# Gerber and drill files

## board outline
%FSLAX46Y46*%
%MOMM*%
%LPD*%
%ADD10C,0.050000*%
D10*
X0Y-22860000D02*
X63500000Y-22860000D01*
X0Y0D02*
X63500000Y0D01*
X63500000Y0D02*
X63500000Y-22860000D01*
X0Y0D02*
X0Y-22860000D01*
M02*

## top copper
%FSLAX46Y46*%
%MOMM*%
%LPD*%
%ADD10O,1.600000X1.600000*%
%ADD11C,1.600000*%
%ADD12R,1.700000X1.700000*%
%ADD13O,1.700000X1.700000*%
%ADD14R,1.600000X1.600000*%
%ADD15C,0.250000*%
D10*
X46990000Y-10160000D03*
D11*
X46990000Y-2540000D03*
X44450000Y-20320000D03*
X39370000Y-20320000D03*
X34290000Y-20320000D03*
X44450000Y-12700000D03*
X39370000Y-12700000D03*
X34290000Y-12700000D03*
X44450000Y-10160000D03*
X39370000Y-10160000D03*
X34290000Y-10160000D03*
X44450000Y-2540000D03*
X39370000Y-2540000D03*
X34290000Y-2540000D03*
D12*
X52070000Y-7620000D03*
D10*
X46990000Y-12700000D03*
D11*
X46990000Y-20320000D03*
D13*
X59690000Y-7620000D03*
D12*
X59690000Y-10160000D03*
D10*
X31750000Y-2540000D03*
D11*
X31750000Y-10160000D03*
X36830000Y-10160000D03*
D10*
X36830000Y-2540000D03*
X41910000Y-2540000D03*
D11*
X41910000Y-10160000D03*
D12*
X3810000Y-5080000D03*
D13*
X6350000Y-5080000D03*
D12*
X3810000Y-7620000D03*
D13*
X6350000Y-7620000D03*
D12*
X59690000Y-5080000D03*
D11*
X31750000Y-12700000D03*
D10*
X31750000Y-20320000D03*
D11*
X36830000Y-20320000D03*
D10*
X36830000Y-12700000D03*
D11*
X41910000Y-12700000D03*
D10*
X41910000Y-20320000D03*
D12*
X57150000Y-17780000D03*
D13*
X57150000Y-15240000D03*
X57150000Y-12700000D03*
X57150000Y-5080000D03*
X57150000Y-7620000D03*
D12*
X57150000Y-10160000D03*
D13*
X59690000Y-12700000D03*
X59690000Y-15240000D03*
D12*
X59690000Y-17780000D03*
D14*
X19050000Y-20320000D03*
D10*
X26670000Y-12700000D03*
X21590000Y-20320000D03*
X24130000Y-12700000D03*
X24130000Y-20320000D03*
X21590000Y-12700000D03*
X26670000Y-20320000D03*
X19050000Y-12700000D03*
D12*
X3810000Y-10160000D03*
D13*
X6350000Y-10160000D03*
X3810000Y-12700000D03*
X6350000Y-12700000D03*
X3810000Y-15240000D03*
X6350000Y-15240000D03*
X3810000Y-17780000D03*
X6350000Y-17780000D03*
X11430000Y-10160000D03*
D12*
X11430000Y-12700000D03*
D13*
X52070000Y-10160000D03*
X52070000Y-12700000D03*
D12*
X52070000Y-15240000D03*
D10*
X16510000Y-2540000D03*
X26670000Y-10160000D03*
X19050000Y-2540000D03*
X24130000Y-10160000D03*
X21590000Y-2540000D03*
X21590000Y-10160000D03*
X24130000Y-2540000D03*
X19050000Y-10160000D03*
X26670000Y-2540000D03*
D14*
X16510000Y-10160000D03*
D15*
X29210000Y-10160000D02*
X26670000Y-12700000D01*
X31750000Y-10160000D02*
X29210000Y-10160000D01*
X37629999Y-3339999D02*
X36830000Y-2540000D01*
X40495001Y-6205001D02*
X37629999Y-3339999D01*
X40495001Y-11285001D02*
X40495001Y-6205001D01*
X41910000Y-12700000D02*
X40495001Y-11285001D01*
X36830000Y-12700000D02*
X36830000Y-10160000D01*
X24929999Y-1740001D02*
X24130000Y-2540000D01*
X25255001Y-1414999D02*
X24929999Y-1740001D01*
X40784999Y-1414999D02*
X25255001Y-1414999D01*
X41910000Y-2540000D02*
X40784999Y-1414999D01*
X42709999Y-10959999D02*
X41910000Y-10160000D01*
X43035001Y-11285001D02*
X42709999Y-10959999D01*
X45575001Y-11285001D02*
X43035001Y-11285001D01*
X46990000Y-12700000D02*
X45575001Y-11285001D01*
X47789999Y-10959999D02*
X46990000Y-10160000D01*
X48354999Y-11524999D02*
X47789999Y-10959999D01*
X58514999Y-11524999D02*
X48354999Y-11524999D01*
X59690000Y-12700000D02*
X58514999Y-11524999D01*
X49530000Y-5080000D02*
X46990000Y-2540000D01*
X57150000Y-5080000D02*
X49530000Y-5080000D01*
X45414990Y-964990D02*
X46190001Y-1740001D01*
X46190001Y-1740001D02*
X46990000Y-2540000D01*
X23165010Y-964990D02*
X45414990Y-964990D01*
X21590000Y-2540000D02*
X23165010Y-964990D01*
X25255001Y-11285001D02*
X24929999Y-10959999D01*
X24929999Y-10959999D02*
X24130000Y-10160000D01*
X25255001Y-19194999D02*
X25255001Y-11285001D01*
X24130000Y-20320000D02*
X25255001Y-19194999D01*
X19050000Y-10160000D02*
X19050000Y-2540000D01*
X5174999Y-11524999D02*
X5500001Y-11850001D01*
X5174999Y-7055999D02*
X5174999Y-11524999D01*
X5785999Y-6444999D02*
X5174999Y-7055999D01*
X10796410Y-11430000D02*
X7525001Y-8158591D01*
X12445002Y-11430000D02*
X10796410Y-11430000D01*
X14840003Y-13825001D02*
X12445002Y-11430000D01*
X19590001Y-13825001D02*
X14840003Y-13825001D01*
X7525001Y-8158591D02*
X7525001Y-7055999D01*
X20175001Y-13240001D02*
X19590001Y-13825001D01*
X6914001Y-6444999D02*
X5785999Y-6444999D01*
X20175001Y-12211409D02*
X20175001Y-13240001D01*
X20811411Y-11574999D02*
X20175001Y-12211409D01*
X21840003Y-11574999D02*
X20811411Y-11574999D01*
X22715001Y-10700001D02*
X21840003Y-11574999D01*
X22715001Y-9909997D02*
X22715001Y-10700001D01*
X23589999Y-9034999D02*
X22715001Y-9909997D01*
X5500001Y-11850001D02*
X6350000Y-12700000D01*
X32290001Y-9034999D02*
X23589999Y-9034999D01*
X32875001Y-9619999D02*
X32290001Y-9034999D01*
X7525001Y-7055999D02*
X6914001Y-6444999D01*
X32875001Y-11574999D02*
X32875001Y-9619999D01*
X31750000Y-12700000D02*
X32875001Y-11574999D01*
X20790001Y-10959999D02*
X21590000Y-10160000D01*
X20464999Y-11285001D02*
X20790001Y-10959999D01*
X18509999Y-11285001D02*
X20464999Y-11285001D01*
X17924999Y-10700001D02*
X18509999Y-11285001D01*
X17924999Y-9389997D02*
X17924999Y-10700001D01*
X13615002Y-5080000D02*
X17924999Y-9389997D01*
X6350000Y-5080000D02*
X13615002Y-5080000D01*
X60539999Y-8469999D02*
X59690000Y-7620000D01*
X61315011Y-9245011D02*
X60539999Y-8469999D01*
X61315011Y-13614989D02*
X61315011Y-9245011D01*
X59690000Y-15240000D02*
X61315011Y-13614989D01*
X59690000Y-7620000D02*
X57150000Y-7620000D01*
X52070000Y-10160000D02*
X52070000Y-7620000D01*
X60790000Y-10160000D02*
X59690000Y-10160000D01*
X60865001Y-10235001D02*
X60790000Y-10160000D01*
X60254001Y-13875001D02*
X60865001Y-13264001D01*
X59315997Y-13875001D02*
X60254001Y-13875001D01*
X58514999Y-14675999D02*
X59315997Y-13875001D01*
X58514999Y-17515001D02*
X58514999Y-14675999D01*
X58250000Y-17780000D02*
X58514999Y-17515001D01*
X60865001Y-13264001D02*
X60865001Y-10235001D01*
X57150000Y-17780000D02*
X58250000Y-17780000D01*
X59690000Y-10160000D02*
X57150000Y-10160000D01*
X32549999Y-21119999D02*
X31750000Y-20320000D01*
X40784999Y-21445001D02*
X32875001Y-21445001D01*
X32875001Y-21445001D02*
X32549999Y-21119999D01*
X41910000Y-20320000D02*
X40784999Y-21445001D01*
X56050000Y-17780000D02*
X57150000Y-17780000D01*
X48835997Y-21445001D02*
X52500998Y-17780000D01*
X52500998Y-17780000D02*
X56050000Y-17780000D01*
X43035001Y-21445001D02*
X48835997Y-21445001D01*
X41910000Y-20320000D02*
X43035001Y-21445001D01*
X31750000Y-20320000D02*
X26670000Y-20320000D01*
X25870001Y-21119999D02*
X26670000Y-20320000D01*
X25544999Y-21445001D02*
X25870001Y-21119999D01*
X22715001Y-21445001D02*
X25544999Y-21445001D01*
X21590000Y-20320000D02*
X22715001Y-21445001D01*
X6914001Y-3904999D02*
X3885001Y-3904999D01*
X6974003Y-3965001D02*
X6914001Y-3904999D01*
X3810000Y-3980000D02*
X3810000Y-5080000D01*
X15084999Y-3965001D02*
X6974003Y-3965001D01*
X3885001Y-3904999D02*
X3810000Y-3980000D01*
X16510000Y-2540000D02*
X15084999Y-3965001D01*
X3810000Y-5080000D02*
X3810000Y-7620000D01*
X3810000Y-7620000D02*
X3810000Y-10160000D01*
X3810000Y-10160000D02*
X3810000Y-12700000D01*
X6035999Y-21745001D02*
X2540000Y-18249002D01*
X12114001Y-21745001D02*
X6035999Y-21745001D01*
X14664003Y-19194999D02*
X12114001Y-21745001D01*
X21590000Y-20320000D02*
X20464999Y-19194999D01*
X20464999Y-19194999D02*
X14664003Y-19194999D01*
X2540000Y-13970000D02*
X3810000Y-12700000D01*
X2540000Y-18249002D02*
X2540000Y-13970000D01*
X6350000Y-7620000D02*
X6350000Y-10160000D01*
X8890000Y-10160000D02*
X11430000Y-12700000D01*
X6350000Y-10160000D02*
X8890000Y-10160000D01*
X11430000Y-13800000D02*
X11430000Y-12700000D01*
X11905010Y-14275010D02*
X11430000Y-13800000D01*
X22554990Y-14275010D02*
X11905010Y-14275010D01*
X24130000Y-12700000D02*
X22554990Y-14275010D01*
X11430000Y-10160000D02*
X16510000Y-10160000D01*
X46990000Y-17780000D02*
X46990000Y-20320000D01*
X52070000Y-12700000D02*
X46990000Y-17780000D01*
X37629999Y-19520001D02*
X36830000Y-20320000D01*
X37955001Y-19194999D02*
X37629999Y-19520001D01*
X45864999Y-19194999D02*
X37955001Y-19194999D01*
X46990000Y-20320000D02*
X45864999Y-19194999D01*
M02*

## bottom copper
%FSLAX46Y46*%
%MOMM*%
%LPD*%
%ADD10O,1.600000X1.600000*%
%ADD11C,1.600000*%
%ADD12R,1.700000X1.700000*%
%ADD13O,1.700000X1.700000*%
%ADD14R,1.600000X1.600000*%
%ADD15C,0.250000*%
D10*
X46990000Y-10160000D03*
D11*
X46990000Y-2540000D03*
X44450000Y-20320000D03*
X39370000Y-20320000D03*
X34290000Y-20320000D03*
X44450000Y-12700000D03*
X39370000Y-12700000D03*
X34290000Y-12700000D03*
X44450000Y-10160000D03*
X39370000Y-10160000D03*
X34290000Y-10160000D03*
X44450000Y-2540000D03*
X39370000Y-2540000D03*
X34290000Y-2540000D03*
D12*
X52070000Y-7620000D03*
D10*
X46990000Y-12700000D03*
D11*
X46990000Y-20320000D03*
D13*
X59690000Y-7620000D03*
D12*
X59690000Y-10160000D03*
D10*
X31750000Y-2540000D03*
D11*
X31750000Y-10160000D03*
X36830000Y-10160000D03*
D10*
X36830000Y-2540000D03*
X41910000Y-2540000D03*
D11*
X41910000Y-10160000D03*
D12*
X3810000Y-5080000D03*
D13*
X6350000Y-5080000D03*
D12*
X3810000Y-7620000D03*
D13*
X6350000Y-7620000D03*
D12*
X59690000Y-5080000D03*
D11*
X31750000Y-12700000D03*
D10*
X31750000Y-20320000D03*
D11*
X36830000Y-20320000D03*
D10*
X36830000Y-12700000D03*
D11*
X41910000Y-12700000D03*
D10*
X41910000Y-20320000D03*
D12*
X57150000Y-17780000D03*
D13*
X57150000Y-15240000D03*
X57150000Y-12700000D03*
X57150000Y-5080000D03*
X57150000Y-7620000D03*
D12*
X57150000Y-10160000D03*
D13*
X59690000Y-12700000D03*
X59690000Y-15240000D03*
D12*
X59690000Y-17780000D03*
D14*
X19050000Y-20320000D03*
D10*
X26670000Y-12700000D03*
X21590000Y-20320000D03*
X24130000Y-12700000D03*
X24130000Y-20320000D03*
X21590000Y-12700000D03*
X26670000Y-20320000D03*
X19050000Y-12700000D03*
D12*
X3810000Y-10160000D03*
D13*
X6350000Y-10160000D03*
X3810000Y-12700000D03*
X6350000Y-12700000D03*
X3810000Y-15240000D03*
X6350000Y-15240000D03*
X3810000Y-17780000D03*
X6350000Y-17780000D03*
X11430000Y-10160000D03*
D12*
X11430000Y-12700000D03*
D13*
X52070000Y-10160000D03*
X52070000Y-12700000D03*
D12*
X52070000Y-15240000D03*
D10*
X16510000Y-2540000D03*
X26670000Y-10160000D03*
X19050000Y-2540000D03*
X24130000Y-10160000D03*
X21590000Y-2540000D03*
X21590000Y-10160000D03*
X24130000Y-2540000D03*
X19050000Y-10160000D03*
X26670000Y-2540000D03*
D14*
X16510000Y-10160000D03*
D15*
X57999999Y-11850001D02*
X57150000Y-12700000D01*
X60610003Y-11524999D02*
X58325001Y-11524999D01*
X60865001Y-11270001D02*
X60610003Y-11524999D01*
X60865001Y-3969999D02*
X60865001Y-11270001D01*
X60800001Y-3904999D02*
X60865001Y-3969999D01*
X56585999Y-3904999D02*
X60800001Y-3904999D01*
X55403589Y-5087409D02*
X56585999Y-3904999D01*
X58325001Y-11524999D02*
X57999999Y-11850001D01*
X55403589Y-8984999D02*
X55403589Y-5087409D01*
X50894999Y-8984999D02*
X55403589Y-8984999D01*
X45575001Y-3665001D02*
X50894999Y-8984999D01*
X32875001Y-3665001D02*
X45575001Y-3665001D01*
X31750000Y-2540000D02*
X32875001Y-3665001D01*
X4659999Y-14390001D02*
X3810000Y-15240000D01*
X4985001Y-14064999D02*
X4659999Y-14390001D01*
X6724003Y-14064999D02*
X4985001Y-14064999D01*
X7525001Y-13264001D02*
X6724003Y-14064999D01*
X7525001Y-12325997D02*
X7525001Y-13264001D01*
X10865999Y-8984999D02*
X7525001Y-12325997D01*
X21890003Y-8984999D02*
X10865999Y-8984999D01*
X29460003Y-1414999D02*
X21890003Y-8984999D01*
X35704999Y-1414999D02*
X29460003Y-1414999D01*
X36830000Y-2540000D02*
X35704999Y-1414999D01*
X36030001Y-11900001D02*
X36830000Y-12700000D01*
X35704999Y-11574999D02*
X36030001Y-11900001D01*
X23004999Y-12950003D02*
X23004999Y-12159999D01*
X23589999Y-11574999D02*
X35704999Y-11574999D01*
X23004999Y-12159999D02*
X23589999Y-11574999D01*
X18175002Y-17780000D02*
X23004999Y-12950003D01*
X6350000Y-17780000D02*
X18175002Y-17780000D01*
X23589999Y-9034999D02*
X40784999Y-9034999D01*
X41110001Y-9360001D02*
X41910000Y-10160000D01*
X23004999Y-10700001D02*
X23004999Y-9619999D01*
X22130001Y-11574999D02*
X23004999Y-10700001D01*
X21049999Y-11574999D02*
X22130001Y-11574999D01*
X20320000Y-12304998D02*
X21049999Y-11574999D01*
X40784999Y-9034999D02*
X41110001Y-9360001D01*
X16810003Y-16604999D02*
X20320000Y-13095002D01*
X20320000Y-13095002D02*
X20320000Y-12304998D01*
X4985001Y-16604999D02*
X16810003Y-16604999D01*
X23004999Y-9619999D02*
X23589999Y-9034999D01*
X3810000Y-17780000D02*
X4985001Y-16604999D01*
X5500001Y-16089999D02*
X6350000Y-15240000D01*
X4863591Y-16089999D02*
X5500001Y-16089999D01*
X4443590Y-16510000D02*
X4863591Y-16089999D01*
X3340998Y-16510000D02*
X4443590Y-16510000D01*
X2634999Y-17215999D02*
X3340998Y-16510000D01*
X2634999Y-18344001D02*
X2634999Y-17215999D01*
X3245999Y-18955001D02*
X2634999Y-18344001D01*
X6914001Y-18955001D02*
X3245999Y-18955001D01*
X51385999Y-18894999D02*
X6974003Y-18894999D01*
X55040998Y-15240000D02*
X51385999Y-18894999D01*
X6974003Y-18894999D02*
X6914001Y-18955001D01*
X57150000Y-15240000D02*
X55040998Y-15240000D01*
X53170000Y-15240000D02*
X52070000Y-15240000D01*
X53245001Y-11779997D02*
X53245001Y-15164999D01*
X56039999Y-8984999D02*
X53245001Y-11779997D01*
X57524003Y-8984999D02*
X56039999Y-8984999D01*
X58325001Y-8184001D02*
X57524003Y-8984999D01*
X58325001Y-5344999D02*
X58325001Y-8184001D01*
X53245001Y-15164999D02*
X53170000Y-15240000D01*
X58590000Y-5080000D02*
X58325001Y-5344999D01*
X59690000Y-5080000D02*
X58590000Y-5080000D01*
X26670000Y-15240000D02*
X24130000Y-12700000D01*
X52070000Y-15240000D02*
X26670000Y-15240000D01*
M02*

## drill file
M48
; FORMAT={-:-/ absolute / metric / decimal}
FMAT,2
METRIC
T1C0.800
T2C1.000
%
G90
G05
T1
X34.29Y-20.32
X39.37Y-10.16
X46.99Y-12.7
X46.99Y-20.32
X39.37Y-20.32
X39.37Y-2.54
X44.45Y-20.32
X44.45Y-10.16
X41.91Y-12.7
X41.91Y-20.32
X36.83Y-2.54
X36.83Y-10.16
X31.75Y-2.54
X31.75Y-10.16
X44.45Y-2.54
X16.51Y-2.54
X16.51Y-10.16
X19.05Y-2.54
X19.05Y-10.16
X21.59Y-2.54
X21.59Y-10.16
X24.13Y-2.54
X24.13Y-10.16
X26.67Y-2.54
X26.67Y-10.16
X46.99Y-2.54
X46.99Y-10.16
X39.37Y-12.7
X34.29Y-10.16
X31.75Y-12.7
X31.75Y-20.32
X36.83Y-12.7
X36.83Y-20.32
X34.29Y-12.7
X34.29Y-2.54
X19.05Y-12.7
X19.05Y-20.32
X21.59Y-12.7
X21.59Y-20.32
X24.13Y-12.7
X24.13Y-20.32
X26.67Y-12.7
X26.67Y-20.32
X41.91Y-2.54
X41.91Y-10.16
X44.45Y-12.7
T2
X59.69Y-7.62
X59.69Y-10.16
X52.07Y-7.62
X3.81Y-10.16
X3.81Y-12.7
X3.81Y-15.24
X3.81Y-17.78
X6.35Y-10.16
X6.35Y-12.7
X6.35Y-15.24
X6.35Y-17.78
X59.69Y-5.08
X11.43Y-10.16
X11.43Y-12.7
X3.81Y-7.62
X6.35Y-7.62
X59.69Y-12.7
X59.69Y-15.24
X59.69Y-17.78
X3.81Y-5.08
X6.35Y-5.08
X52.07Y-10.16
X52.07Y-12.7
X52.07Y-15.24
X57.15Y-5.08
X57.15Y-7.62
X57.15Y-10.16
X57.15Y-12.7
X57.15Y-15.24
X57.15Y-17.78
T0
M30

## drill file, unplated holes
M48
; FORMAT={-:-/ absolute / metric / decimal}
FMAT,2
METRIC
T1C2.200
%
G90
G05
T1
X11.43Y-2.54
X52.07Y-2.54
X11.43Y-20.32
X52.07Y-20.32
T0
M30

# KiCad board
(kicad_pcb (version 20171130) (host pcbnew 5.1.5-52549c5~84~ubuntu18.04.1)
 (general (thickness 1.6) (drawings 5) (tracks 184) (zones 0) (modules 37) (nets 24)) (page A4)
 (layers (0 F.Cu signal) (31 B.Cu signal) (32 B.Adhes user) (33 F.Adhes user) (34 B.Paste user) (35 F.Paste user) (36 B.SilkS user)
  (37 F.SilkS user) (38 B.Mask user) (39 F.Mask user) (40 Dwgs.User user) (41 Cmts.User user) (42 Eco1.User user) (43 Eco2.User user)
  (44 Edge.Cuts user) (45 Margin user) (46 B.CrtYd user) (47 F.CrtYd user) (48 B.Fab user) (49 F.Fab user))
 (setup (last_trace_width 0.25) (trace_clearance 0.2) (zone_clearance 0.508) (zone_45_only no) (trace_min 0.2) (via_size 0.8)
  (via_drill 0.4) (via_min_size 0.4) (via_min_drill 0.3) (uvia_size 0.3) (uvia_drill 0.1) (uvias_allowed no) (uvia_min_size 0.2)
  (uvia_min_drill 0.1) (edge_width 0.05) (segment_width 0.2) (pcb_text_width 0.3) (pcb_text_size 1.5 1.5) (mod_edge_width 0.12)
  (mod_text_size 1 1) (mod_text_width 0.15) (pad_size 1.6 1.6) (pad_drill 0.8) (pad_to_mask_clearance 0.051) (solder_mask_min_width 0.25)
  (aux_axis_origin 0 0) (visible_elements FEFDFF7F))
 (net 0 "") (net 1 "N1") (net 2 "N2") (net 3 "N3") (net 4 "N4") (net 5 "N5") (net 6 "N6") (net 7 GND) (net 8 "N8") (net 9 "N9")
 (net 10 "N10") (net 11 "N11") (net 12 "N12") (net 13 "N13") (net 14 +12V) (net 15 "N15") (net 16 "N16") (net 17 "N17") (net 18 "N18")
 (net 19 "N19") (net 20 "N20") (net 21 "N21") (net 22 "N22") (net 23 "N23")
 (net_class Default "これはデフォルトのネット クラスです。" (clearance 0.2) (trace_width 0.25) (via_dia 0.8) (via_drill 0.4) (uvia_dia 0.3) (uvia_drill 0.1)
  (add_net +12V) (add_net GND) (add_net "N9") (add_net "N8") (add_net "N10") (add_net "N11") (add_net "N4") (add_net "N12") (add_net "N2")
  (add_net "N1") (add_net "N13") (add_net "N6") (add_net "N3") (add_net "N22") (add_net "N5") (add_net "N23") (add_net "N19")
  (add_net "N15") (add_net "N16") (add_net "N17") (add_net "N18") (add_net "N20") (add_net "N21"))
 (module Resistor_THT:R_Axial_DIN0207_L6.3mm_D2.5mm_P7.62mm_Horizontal (layer F.Cu) (at 46.99 2.54 270)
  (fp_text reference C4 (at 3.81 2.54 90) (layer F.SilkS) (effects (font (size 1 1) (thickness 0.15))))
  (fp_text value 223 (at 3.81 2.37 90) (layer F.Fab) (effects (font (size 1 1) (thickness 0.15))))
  (pad 2 thru_hole oval (at 7.62 0 270) (size 1.6 1.6) (drill 0.8) (layers *.Cu *.Mask) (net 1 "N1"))
  (pad 1 thru_hole circle (at 0 0 270) (size 1.6 1.6) (drill 0.8) (layers *.Cu *.Mask) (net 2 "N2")))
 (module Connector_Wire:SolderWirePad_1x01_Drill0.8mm (layer F.Cu) (at 44.45 20.32)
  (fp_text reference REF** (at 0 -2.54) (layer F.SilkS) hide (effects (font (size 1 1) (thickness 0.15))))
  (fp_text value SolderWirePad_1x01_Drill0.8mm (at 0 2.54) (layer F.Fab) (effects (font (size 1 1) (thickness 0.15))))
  (pad 1 thru_hole circle (at 0 0) (size 1.6 1.6) (drill 0.8) (layers *.Cu *.Mask)))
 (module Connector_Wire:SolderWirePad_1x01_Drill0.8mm (layer F.Cu) (at 39.37 20.32)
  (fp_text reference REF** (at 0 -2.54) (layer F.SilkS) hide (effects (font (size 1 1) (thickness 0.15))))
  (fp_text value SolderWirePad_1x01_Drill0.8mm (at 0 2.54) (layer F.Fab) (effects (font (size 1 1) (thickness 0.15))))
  (pad 1 thru_hole circle (at 0 0) (size 1.6 1.6) (drill 0.8) (layers *.Cu *.Mask)))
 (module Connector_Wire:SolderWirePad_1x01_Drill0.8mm (layer F.Cu) (at 34.29 20.32)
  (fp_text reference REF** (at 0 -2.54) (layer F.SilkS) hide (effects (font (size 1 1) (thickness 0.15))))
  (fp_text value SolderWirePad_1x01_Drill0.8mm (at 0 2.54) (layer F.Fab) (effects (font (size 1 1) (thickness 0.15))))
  (pad 1 thru_hole circle (at 0 0) (size 1.6 1.6) (drill 0.8) (layers *.Cu *.Mask)))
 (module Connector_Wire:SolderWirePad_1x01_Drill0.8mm (layer F.Cu) (at 44.45 12.7)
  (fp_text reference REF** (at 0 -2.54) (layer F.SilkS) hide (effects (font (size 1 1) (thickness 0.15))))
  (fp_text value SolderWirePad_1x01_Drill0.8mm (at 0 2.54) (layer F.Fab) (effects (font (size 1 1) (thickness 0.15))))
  (pad 1 thru_hole circle (at 0 0) (size 1.6 1.6) (drill 0.8) (layers *.Cu *.Mask)))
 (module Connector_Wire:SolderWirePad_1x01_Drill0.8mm (layer F.Cu) (at 39.37 12.7)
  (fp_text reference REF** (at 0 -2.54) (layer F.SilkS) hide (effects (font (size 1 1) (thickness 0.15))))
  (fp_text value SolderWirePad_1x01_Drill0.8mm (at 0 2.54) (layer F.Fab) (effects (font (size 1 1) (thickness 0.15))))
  (pad 1 thru_hole circle (at 0 0) (size 1.6 1.6) (drill 0.8) (layers *.Cu *.Mask)))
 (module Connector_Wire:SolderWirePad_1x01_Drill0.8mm (layer F.Cu) (at 34.29 12.7)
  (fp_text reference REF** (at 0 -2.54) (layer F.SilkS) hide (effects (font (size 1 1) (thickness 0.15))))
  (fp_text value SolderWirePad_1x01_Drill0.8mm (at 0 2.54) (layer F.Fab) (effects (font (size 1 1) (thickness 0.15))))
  (pad 1 thru_hole circle (at 0 0) (size 1.6 1.6) (drill 0.8) (layers *.Cu *.Mask)))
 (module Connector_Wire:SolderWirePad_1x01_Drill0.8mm (layer F.Cu) (at 44.45 10.16)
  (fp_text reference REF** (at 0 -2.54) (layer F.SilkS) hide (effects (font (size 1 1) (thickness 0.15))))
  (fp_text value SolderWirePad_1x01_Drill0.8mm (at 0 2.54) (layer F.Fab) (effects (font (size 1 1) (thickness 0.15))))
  (pad 1 thru_hole circle (at 0 0) (size 1.6 1.6) (drill 0.8) (layers *.Cu *.Mask)))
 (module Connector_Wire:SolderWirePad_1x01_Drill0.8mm (layer F.Cu) (at 39.37 10.16)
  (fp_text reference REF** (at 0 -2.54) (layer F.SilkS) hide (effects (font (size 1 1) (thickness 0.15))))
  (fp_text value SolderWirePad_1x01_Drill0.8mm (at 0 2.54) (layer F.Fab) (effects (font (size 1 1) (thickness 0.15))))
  (pad 1 thru_hole circle (at 0 0) (size 1.6 1.6) (drill 0.8) (layers *.Cu *.Mask)))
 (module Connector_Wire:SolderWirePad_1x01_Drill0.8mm (layer F.Cu) (at 34.29 10.16)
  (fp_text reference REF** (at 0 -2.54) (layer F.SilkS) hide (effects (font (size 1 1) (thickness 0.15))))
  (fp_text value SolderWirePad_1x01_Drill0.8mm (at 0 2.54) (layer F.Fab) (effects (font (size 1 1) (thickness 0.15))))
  (pad 1 thru_hole circle (at 0 0) (size 1.6 1.6) (drill 0.8) (layers *.Cu *.Mask)))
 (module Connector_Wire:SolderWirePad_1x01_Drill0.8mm (layer F.Cu) (at 44.45 2.54)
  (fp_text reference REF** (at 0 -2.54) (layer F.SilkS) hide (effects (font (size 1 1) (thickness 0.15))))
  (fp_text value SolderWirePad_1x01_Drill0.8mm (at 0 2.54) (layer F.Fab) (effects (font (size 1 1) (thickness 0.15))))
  (pad 1 thru_hole circle (at 0 0) (size 1.6 1.6) (drill 0.8) (layers *.Cu *.Mask)))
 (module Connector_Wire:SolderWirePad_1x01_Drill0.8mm (layer F.Cu) (at 39.37 2.54)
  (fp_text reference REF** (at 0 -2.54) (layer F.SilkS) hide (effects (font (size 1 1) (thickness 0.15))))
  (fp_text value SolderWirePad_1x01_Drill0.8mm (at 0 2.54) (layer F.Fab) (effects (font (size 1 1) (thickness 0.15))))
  (pad 1 thru_hole circle (at 0 0) (size 1.6 1.6) (drill 0.8) (layers *.Cu *.Mask)))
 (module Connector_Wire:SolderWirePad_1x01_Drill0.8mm (layer F.Cu) (at 34.29 2.54)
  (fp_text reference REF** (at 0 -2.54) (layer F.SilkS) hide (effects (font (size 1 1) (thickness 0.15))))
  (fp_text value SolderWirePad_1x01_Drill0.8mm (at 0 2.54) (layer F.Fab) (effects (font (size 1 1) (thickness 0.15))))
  (pad 1 thru_hole circle (at 0 0) (size 1.6 1.6) (drill 0.8) (layers *.Cu *.Mask)))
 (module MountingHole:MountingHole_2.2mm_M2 (layer F.Cu) (at 52.07 20.32)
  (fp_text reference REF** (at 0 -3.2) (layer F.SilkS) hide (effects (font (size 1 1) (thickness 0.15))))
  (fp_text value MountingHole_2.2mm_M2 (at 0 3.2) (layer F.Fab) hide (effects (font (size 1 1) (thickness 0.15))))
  (pad 1 np_thru_hole circle (at 0 0) (size 2.2 2.2) (drill 2.2) (layers *.Cu *.Mask)))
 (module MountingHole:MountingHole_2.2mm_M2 (layer F.Cu) (at 11.43 20.32)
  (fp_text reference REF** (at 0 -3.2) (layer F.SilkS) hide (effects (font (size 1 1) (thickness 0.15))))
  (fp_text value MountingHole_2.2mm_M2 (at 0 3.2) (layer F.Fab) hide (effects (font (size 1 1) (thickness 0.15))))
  (pad 1 np_thru_hole circle (at 0 0) (size 2.2 2.2) (drill 2.2) (layers *.Cu *.Mask)))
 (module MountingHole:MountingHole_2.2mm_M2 (layer F.Cu) (at 52.07 2.54)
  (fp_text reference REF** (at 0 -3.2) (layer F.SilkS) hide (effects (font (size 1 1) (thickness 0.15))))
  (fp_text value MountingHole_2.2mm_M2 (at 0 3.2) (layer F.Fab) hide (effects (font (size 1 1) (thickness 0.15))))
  (pad 1 np_thru_hole circle (at 0 0) (size 2.2 2.2) (drill 2.2) (layers *.Cu *.Mask)))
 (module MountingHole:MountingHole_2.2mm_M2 (layer F.Cu) (at 11.43 2.54)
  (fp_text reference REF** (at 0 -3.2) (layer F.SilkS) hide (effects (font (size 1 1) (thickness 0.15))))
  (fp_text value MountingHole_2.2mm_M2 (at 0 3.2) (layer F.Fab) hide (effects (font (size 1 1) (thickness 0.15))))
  (pad 1 np_thru_hole circle (at 0 0) (size 2.2 2.2) (drill 2.2) (layers *.Cu *.Mask)))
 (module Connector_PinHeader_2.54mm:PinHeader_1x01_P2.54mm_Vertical (layer F.Cu) (at 52.07 7.62)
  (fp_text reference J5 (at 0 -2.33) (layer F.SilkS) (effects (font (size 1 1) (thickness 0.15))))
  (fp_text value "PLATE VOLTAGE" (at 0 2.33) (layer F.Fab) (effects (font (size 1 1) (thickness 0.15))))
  (pad 1 thru_hole rect (at 0 0) (size 1.7 1.7) (drill 1) (layers *.Cu *.Mask) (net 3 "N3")))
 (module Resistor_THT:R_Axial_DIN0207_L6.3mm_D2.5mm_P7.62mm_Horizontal (layer F.Cu) (at 46.99 20.32 90)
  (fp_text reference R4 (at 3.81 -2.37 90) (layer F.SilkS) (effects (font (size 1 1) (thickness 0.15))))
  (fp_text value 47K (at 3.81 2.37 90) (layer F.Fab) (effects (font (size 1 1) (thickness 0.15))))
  (pad 2 thru_hole oval (at 7.62 0 90) (size 1.6 1.6) (drill 0.8) (layers *.Cu *.Mask) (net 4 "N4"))
  (pad 1 thru_hole circle (at 0 0 90) (size 1.6 1.6) (drill 0.8) (layers *.Cu *.Mask) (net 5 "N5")))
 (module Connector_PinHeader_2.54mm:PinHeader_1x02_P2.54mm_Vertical (layer F.Cu) (at 59.69 10.16 180)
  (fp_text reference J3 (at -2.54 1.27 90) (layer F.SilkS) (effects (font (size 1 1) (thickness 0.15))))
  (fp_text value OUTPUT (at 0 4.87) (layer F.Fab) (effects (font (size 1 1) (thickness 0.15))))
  (pad 2 thru_hole oval (at 0 2.54 180) (size 1.7 1.7) (drill 1) (layers *.Cu *.Mask) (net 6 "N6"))
  (pad 1 thru_hole rect (at 0 0 180) (size 1.7 1.7) (drill 1) (layers *.Cu *.Mask) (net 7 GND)))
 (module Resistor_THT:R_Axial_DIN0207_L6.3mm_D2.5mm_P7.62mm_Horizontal (layer F.Cu) (at 31.75 10.16 90)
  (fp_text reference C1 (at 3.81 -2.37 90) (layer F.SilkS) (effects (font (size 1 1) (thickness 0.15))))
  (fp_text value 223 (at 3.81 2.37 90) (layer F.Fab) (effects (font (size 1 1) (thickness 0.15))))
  (pad 2 thru_hole oval (at 7.62 0 90) (size 1.6 1.6) (drill 0.8) (layers *.Cu *.Mask) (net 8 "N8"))
  (pad 1 thru_hole circle (at 0 0 90) (size 1.6 1.6) (drill 0.8) (layers *.Cu *.Mask) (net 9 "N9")))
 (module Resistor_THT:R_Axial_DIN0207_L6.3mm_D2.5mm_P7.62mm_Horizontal (layer F.Cu) (at 36.83 10.16 90)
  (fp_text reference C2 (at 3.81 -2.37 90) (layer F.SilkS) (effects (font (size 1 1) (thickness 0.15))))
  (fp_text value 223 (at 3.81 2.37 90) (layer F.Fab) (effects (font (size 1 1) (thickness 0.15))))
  (pad 1 thru_hole circle (at 0 0 90) (size 1.6 1.6) (drill 0.8) (layers *.Cu *.Mask) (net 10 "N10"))
  (pad 2 thru_hole oval (at 7.62 0 90) (size 1.6 1.6) (drill 0.8) (layers *.Cu *.Mask) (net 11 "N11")))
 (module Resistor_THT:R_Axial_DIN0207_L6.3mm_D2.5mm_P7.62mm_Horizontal (layer F.Cu) (at 41.91 10.16 90)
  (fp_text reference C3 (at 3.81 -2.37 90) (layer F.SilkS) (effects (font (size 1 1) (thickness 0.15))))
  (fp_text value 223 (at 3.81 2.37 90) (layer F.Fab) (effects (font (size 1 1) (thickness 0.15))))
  (pad 2 thru_hole oval (at 7.62 0 90) (size 1.6 1.6) (drill 0.8) (layers *.Cu *.Mask) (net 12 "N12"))
  (pad 1 thru_hole circle (at 0 0 90) (size 1.6 1.6) (drill 0.8) (layers *.Cu *.Mask) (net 4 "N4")))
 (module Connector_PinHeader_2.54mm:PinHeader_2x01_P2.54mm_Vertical (layer F.Cu) (at 3.81 5.08)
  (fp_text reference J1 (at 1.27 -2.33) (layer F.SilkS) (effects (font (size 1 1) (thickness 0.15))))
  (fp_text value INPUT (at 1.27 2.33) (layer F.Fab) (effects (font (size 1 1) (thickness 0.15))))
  (pad 1 thru_hole rect (at 0 0) (size 1.7 1.7) (drill 1) (layers *.Cu *.Mask) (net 7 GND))
  (pad 2 thru_hole oval (at 2.54 0) (size 1.7 1.7) (drill 1) (layers *.Cu *.Mask) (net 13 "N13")))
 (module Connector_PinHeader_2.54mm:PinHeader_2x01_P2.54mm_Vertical (layer F.Cu) (at 3.81 7.62)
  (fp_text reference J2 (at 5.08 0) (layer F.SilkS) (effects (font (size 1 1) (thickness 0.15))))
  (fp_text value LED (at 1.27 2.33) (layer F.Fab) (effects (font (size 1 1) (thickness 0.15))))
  (pad 1 thru_hole rect (at 0 0) (size 1.7 1.7) (drill 1) (layers *.Cu *.Mask) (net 7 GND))
  (pad 2 thru_hole oval (at 2.54 0) (size 1.7 1.7) (drill 1) (layers *.Cu *.Mask) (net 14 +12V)))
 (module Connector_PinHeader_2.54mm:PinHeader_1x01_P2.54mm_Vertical (layer F.Cu) (at 59.69 5.08 180)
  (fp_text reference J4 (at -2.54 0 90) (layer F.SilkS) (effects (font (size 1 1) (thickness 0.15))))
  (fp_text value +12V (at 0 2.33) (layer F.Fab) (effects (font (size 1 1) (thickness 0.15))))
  (pad 1 thru_hole rect (at 0 0 180) (size 1.7 1.7) (drill 1) (layers *.Cu *.Mask) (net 14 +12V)))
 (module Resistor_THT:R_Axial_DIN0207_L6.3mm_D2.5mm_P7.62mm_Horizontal (layer F.Cu) (at 31.75 12.7 270)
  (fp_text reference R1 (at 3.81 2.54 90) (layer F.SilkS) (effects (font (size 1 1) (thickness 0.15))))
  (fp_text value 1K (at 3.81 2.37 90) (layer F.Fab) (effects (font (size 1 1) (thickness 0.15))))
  (pad 1 thru_hole circle (at 0 0 270) (size 1.6 1.6) (drill 0.8) (layers *.Cu *.Mask) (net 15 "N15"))
  (pad 2 thru_hole oval (at 7.62 0 270) (size 1.6 1.6) (drill 0.8) (layers *.Cu *.Mask) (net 7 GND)))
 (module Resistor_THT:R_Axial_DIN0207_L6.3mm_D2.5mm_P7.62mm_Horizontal (layer F.Cu) (at 36.83 20.32 90)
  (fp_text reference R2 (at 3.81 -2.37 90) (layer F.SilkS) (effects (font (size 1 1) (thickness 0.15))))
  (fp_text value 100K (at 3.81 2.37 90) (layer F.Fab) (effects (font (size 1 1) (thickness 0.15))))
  (pad 1 thru_hole circle (at 0 0 90) (size 1.6 1.6) (drill 0.8) (layers *.Cu *.Mask) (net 5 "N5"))
  (pad 2 thru_hole oval (at 7.62 0 90) (size 1.6 1.6) (drill 0.8) (layers *.Cu *.Mask) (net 10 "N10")))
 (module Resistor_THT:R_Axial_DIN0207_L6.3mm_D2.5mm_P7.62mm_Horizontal (layer F.Cu) (at 41.91 12.7 270)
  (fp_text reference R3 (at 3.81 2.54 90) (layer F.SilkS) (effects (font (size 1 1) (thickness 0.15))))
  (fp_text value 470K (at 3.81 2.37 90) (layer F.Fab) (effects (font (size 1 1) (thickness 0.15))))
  (pad 1 thru_hole circle (at 0 0 270) (size 1.6 1.6) (drill 0.8) (layers *.Cu *.Mask) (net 11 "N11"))
  (pad 2 thru_hole oval (at 7.62 0 270) (size 1.6 1.6) (drill 0.8) (layers *.Cu *.Mask) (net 7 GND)))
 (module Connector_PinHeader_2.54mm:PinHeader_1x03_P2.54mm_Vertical (layer F.Cu) (at 57.15 17.78 180)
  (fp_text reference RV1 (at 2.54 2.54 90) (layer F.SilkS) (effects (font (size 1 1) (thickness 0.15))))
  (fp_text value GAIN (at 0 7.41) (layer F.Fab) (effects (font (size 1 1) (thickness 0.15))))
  (pad 1 thru_hole rect (at 0 0 180) (size 1.7 1.7) (drill 1) (layers *.Cu *.Mask) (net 7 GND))
  (pad 2 thru_hole oval (at 0 2.54 180) (size 1.7 1.7) (drill 1) (layers *.Cu *.Mask) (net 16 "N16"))
  (pad 3 thru_hole oval (at 0 5.08 180) (size 1.7 1.7) (drill 1) (layers *.Cu *.Mask) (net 8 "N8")))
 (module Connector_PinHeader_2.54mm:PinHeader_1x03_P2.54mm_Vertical (layer F.Cu) (at 57.15 10.16 180)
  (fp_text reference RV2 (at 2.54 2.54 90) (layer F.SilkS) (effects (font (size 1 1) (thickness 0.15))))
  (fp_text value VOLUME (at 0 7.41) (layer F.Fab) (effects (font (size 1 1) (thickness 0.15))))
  (pad 3 thru_hole oval (at 0 5.08 180) (size 1.7 1.7) (drill 1) (layers *.Cu *.Mask) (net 2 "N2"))
  (pad 2 thru_hole oval (at 0 2.54 180) (size 1.7 1.7) (drill 1) (layers *.Cu *.Mask) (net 6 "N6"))
  (pad 1 thru_hole rect (at 0 0 180) (size 1.7 1.7) (drill 1) (layers *.Cu *.Mask) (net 7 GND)))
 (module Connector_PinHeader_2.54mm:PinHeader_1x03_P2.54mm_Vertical (layer F.Cu) (at 59.69 17.78 180)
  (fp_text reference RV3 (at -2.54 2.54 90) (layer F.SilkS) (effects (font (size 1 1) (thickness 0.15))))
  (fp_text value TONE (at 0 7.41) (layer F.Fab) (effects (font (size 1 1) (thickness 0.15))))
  (pad 3 thru_hole oval (at 0 5.08 180) (size 1.7 1.7) (drill 1) (layers *.Cu *.Mask) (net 1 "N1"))
  (pad 2 thru_hole oval (at 0 2.54 180) (size 1.7 1.7) (drill 1) (layers *.Cu *.Mask) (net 6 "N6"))
  (pad 1 thru_hole rect (at 0 0 180) (size 1.7 1.7) (drill 1) (layers *.Cu *.Mask) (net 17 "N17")))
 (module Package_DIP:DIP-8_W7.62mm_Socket (layer F.Cu) (at 19.05 20.32 90)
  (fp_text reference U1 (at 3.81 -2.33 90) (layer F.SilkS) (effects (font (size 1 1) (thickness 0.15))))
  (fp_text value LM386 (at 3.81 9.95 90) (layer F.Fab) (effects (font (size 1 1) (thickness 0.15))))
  (pad 1 thru_hole rect (at 0 0 90) (size 1.6 1.6) (drill 0.8) (layers *.Cu *.Mask) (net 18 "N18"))
  (pad 5 thru_hole oval (at 7.62 7.62 90) (size 1.6 1.6) (drill 0.8) (layers *.Cu *.Mask) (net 9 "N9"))
  (pad 2 thru_hole oval (at 0 2.54 90) (size 1.6 1.6) (drill 0.8) (layers *.Cu *.Mask) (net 7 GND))
  (pad 6 thru_hole oval (at 7.62 5.08 90) (size 1.6 1.6) (drill 0.8) (layers *.Cu *.Mask) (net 14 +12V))
  (pad 3 thru_hole oval (at 0 5.08 90) (size 1.6 1.6) (drill 0.8) (layers *.Cu *.Mask) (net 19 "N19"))
  (pad 7 thru_hole oval (at 7.62 2.54 90) (size 1.6 1.6) (drill 0.8) (layers *.Cu *.Mask) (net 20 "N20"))
  (pad 4 thru_hole oval (at 0 7.62 90) (size 1.6 1.6) (drill 0.8) (layers *.Cu *.Mask) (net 7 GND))
  (pad 8 thru_hole oval (at 7.62 0 90) (size 1.6 1.6) (drill 0.8) (layers *.Cu *.Mask) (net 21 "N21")))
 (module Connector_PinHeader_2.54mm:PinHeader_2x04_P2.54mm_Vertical (layer F.Cu) (at 3.81 10.16)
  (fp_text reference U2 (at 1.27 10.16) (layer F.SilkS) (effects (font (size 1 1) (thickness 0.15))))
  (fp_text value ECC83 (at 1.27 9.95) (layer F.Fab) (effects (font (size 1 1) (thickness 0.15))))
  (pad 4 thru_hole rect (at 0 0) (size 1.7 1.7) (drill 1) (layers *.Cu *.Mask) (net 7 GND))
  (pad 5 thru_hole oval (at 2.54 0) (size 1.7 1.7) (drill 1) (layers *.Cu *.Mask) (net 14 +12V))
  (pad 3 thru_hole oval (at 0 2.54) (size 1.7 1.7) (drill 1) (layers *.Cu *.Mask) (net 7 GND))
  (pad 8 thru_hole oval (at 2.54 2.54) (size 1.7 1.7) (drill 1) (layers *.Cu *.Mask) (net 15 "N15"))
  (pad 2 thru_hole oval (at 0 5.08) (size 1.7 1.7) (drill 1) (layers *.Cu *.Mask) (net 11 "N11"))
  (pad 7 thru_hole oval (at 2.54 5.08) (size 1.7 1.7) (drill 1) (layers *.Cu *.Mask) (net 16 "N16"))
  (pad 1 thru_hole oval (at 0 7.62) (size 1.7 1.7) (drill 1) (layers *.Cu *.Mask) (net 4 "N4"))
  (pad 6 thru_hole oval (at 2.54 7.62) (size 1.7 1.7) (drill 1) (layers *.Cu *.Mask) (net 10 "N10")))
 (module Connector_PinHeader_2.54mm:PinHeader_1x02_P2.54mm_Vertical (layer F.Cu) (at 11.43 12.7 180)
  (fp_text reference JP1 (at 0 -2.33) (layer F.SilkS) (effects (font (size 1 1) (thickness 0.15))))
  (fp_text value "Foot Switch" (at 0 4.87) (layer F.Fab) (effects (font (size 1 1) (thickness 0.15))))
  (pad 2 thru_hole oval (at 0 2.54 180) (size 1.7 1.7) (drill 1) (layers *.Cu *.Mask) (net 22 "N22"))
  (pad 1 thru_hole rect (at 0 0 180) (size 1.7 1.7) (drill 1) (layers *.Cu *.Mask) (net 14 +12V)))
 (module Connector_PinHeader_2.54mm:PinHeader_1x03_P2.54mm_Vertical (layer F.Cu) (at 52.07 15.24 180)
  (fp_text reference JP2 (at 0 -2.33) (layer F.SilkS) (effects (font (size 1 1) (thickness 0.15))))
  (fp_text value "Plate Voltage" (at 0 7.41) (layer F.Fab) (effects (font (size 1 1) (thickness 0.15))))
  (pad 3 thru_hole oval (at 0 5.08 180) (size 1.7 1.7) (drill 1) (layers *.Cu *.Mask) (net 3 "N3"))
  (pad 2 thru_hole oval (at 0 2.54 180) (size 1.7 1.7) (drill 1) (layers *.Cu *.Mask) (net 5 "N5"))
  (pad 1 thru_hole rect (at 0 0 180) (size 1.7 1.7) (drill 1) (layers *.Cu *.Mask) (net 14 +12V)))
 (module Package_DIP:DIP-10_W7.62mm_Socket (layer F.Cu) (at 16.51 10.16 90)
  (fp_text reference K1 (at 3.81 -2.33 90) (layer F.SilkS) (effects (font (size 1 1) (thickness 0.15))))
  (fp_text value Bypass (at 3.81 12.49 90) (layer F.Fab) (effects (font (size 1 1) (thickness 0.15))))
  (pad 10 thru_hole oval (at 7.62 0 90) (size 1.6 1.6) (drill 0.8) (layers *.Cu *.Mask) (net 7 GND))
  (pad 5 thru_hole oval (at 0 10.16 90) (size 1.6 1.6) (drill 0.8) (layers *.Cu *.Mask))
  (pad 9 thru_hole oval (at 7.62 2.54 90) (size 1.6 1.6) (drill 0.8) (layers *.Cu *.Mask) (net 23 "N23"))
  (pad 4 thru_hole oval (at 0 7.62 90) (size 1.6 1.6) (drill 0.8) (layers *.Cu *.Mask) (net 19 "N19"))
  (pad 8 thru_hole oval (at 7.62 5.08 90) (size 1.6 1.6) (drill 0.8) (layers *.Cu *.Mask) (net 2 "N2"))
  (pad 3 thru_hole oval (at 0 5.08 90) (size 1.6 1.6) (drill 0.8) (layers *.Cu *.Mask) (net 13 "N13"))
  (pad 7 thru_hole oval (at 7.62 7.62 90) (size 1.6 1.6) (drill 0.8) (layers *.Cu *.Mask) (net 12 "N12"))
  (pad 2 thru_hole oval (at 0 2.54 90) (size 1.6 1.6) (drill 0.8) (layers *.Cu *.Mask) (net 23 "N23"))
  (pad 6 thru_hole oval (at 7.62 10.16 90) (size 1.6 1.6) (drill 0.8) (layers *.Cu *.Mask))
  (pad 1 thru_hole rect (at 0 0 90) (size 1.6 1.6) (drill 0.8) (layers *.Cu *.Mask) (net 22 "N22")))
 (gr_line (start 0 22.86) (end 63.5 22.86) (layer Edge.Cuts) (width 0.05))
 (gr_line (start 0 0) (end 63.5 0) (layer Edge.Cuts) (width 0.05))
 (gr_line (start 63.5 0) (end 63.5 22.86) (layer Edge.Cuts) (width 0.05))
 (gr_line (start 0 0) (end 0 22.86) (layer Edge.Cuts) (width 0.05))
 (segment (start 57.999999 11.850001) (end 57.15 12.7) (width 0.25) (layer B.Cu) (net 8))
 (segment (start 60.610003 11.524999) (end 58.325001 11.524999) (width 0.25) (layer B.Cu) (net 8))
 (segment (start 60.865001 11.270001) (end 60.610003 11.524999) (width 0.25) (layer B.Cu) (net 8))
 (segment (start 60.865001 3.969999) (end 60.865001 11.270001) (width 0.25) (layer B.Cu) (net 8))
 (segment (start 60.800001 3.904999) (end 60.865001 3.969999) (width 0.25) (layer B.Cu) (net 8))
 (segment (start 56.585999 3.904999) (end 60.800001 3.904999) (width 0.25) (layer B.Cu) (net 8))
 (segment (start 55.403589 5.087409) (end 56.585999 3.904999) (width 0.25) (layer B.Cu) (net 8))
 (segment (start 58.325001 11.524999) (end 57.999999 11.850001) (width 0.25) (layer B.Cu) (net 8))
 (segment (start 55.403589 8.984999) (end 55.403589 5.087409) (width 0.25) (layer B.Cu) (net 8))
 (segment (start 50.894999 8.984999) (end 55.403589 8.984999) (width 0.25) (layer B.Cu) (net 8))
 (segment (start 45.575001 3.665001) (end 50.894999 8.984999) (width 0.25) (layer B.Cu) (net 8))
 (segment (start 32.875001 3.665001) (end 45.575001 3.665001) (width 0.25) (layer B.Cu) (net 8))
 (segment (start 31.75 2.54) (end 32.875001 3.665001) (width 0.25) (layer B.Cu) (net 8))
 (segment (start 29.21 10.16) (end 26.67 12.7) (width 0.25) (layer F.Cu) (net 9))
 (segment (start 31.75 10.16) (end 29.21 10.16) (width 0.25) (layer F.Cu) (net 9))
 (segment (start 37.629999 3.339999) (end 36.83 2.54) (width 0.25) (layer F.Cu) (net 11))
 (segment (start 40.495001 6.205001) (end 37.629999 3.339999) (width 0.25) (layer F.Cu) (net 11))
 (segment (start 40.495001 11.285001) (end 40.495001 6.205001) (width 0.25) (layer F.Cu) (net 11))
 (segment (start 41.91 12.7) (end 40.495001 11.285001) (width 0.25) (layer F.Cu) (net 11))
 (segment (start 4.659999 14.390001) (end 3.81 15.24) (width 0.25) (layer B.Cu) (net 11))
 (segment (start 4.985001 14.064999) (end 4.659999 14.390001) (width 0.25) (layer B.Cu) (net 11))
 (segment (start 6.724003 14.064999) (end 4.985001 14.064999) (width 0.25) (layer B.Cu) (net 11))
 (segment (start 7.525001 13.264001) (end 6.724003 14.064999) (width 0.25) (layer B.Cu) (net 11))
 (segment (start 7.525001 12.325997) (end 7.525001 13.264001) (width 0.25) (layer B.Cu) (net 11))
 (segment (start 10.865999 8.984999) (end 7.525001 12.325997) (width 0.25) (layer B.Cu) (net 11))
 (segment (start 21.890003 8.984999) (end 10.865999 8.984999) (width 0.25) (layer B.Cu) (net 11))
 (segment (start 29.460003 1.414999) (end 21.890003 8.984999) (width 0.25) (layer B.Cu) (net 11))
 (segment (start 35.704999 1.414999) (end 29.460003 1.414999) (width 0.25) (layer B.Cu) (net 11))
 (segment (start 36.83 2.54) (end 35.704999 1.414999) (width 0.25) (layer B.Cu) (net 11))
 (segment (start 36.83 12.7) (end 36.83 10.16) (width 0.25) (layer F.Cu) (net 10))
 (segment (start 36.030001 11.900001) (end 36.83 12.7) (width 0.25) (layer B.Cu) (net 10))
 (segment (start 35.704999 11.574999) (end 36.030001 11.900001) (width 0.25) (layer B.Cu) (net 10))
 (segment (start 23.004999 12.950003) (end 23.004999 12.159999) (width 0.25) (layer B.Cu) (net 10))
 (segment (start 23.589999 11.574999) (end 35.704999 11.574999) (width 0.25) (layer B.Cu) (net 10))
 (segment (start 23.004999 12.159999) (end 23.589999 11.574999) (width 0.25) (layer B.Cu) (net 10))
 (segment (start 18.175002 17.78) (end 23.004999 12.950003) (width 0.25) (layer B.Cu) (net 10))
 (segment (start 6.35 17.78) (end 18.175002 17.78) (width 0.25) (layer B.Cu) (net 10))
 (segment (start 24.929999 1.740001) (end 24.13 2.54) (width 0.25) (layer F.Cu) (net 12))
 (segment (start 25.255001 1.414999) (end 24.929999 1.740001) (width 0.25) (layer F.Cu) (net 12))
 (segment (start 40.784999 1.414999) (end 25.255001 1.414999) (width 0.25) (layer F.Cu) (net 12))
 (segment (start 41.91 2.54) (end 40.784999 1.414999) (width 0.25) (layer F.Cu) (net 12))
 (segment (start 42.709999 10.959999) (end 41.91 10.16) (width 0.25) (layer F.Cu) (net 4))
 (segment (start 43.035001 11.285001) (end 42.709999 10.959999) (width 0.25) (layer F.Cu) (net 4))
 (segment (start 45.575001 11.285001) (end 43.035001 11.285001) (width 0.25) (layer F.Cu) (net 4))
 (segment (start 46.99 12.7) (end 45.575001 11.285001) (width 0.25) (layer F.Cu) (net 4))
 (segment (start 23.589999 9.034999) (end 40.784999 9.034999) (width 0.25) (layer B.Cu) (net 4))
 (segment (start 41.110001 9.360001) (end 41.91 10.16) (width 0.25) (layer B.Cu) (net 4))
 (segment (start 23.004999 10.700001) (end 23.004999 9.619999) (width 0.25) (layer B.Cu) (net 4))
 (segment (start 22.130001 11.574999) (end 23.004999 10.700001) (width 0.25) (layer B.Cu) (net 4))
 (segment (start 21.049999 11.574999) (end 22.130001 11.574999) (width 0.25) (layer B.Cu) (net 4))
 (segment (start 20.32 12.304998) (end 21.049999 11.574999) (width 0.25) (layer B.Cu) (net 4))
 (segment (start 40.784999 9.034999) (end 41.110001 9.360001) (width 0.25) (layer B.Cu) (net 4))
 (segment (start 16.810003 16.604999) (end 20.32 13.095002) (width 0.25) (layer B.Cu) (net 4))
 (segment (start 20.32 13.095002) (end 20.32 12.304998) (width 0.25) (layer B.Cu) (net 4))
 (segment (start 4.985001 16.604999) (end 16.810003 16.604999) (width 0.25) (layer B.Cu) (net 4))
 (segment (start 23.004999 9.619999) (end 23.589999 9.034999) (width 0.25) (layer B.Cu) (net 4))
 (segment (start 3.81 17.78) (end 4.985001 16.604999) (width 0.25) (layer B.Cu) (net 4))
 (segment (start 47.789999 10.959999) (end 46.99 10.16) (width 0.25) (layer F.Cu) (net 1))
 (segment (start 48.354999 11.524999) (end 47.789999 10.959999) (width 0.25) (layer F.Cu) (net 1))
 (segment (start 58.514999 11.524999) (end 48.354999 11.524999) (width 0.25) (layer F.Cu) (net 1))
 (segment (start 59.69 12.7) (end 58.514999 11.524999) (width 0.25) (layer F.Cu) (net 1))
 (segment (start 49.53 5.08) (end 46.99 2.54) (width 0.25) (layer F.Cu) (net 2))
 (segment (start 57.15 5.08) (end 49.53 5.08) (width 0.25) (layer F.Cu) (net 2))
 (segment (start 45.41499 0.96499) (end 46.190001 1.740001) (width 0.25) (layer F.Cu) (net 2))
 (segment (start 46.190001 1.740001) (end 46.99 2.54) (width 0.25) (layer F.Cu) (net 2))
 (segment (start 23.16501 0.96499) (end 45.41499 0.96499) (width 0.25) (layer F.Cu) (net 2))
 (segment (start 21.59 2.54) (end 23.16501 0.96499) (width 0.25) (layer F.Cu) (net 2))
 (segment (start 25.255001 11.285001) (end 24.929999 10.959999) (width 0.25) (layer F.Cu) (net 19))
 (segment (start 24.929999 10.959999) (end 24.13 10.16) (width 0.25) (layer F.Cu) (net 19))
 (segment (start 25.255001 19.194999) (end 25.255001 11.285001) (width 0.25) (layer F.Cu) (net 19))
 (segment (start 24.13 20.32) (end 25.255001 19.194999) (width 0.25) (layer F.Cu) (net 19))
 (segment (start 19.05 10.16) (end 19.05 2.54) (width 0.25) (layer F.Cu) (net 23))
 (segment (start 5.174999 11.524999) (end 5.500001 11.850001) (width 0.25) (layer F.Cu) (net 15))
 (segment (start 5.174999 7.055999) (end 5.174999 11.524999) (width 0.25) (layer F.Cu) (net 15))
 (segment (start 5.785999 6.444999) (end 5.174999 7.055999) (width 0.25) (layer F.Cu) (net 15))
 (segment (start 10.79641 11.43) (end 7.525001 8.158591) (width 0.25) (layer F.Cu) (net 15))
 (segment (start 12.445002 11.43) (end 10.79641 11.43) (width 0.25) (layer F.Cu) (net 15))
 (segment (start 14.840003 13.825001) (end 12.445002 11.43) (width 0.25) (layer F.Cu) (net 15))
 (segment (start 19.590001 13.825001) (end 14.840003 13.825001) (width 0.25) (layer F.Cu) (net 15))
 (segment (start 7.525001 8.158591) (end 7.525001 7.055999) (width 0.25) (layer F.Cu) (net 15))
 (segment (start 20.175001 13.240001) (end 19.590001 13.825001) (width 0.25) (layer F.Cu) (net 15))
 (segment (start 6.914001 6.444999) (end 5.785999 6.444999) (width 0.25) (layer F.Cu) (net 15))
 (segment (start 20.175001 12.211409) (end 20.175001 13.240001) (width 0.25) (layer F.Cu) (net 15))
 (segment (start 20.811411 11.574999) (end 20.175001 12.211409) (width 0.25) (layer F.Cu) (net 15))
 (segment (start 21.840003 11.574999) (end 20.811411 11.574999) (width 0.25) (layer F.Cu) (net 15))
 (segment (start 22.715001 10.700001) (end 21.840003 11.574999) (width 0.25) (layer F.Cu) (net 15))
 (segment (start 22.715001 9.909997) (end 22.715001 10.700001) (width 0.25) (layer F.Cu) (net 15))
 (segment (start 23.589999 9.034999) (end 22.715001 9.909997) (width 0.25) (layer F.Cu) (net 15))
 (segment (start 5.500001 11.850001) (end 6.35 12.7) (width 0.25) (layer F.Cu) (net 15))
 (segment (start 32.290001 9.034999) (end 23.589999 9.034999) (width 0.25) (layer F.Cu) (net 15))
 (segment (start 32.875001 9.619999) (end 32.290001 9.034999) (width 0.25) (layer F.Cu) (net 15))
 (segment (start 7.525001 7.055999) (end 6.914001 6.444999) (width 0.25) (layer F.Cu) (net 15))
 (segment (start 32.875001 11.574999) (end 32.875001 9.619999) (width 0.25) (layer F.Cu) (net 15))
 (segment (start 31.75 12.7) (end 32.875001 11.574999) (width 0.25) (layer F.Cu) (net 15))
 (segment (start 5.500001 16.089999) (end 6.35 15.24) (width 0.25) (layer B.Cu) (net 16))
 (segment (start 4.863591 16.089999) (end 5.500001 16.089999) (width 0.25) (layer B.Cu) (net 16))
 (segment (start 4.44359 16.51) (end 4.863591 16.089999) (width 0.25) (layer B.Cu) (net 16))
 (segment (start 3.340998 16.51) (end 4.44359 16.51) (width 0.25) (layer B.Cu) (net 16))
 (segment (start 2.634999 17.215999) (end 3.340998 16.51) (width 0.25) (layer B.Cu) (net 16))
 (segment (start 2.634999 18.344001) (end 2.634999 17.215999) (width 0.25) (layer B.Cu) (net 16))
 (segment (start 3.245999 18.955001) (end 2.634999 18.344001) (width 0.25) (layer B.Cu) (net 16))
 (segment (start 6.914001 18.955001) (end 3.245999 18.955001) (width 0.25) (layer B.Cu) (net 16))
 (segment (start 51.385999 18.894999) (end 6.974003 18.894999) (width 0.25) (layer B.Cu) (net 16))
 (segment (start 55.040998 15.24) (end 51.385999 18.894999) (width 0.25) (layer B.Cu) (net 16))
 (segment (start 6.974003 18.894999) (end 6.914001 18.955001) (width 0.25) (layer B.Cu) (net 16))
 (segment (start 57.15 15.24) (end 55.040998 15.24) (width 0.25) (layer B.Cu) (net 16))
 (segment (start 20.790001 10.959999) (end 21.59 10.16) (width 0.25) (layer F.Cu) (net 13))
 (segment (start 20.464999 11.285001) (end 20.790001 10.959999) (width 0.25) (layer F.Cu) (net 13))
 (segment (start 18.509999 11.285001) (end 20.464999 11.285001) (width 0.25) (layer F.Cu) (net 13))
 (segment (start 17.924999 10.700001) (end 18.509999 11.285001) (width 0.25) (layer F.Cu) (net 13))
 (segment (start 17.924999 9.389997) (end 17.924999 10.700001) (width 0.25) (layer F.Cu) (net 13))
 (segment (start 13.615002 5.08) (end 17.924999 9.389997) (width 0.25) (layer F.Cu) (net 13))
 (segment (start 6.35 5.08) (end 13.615002 5.08) (width 0.25) (layer F.Cu) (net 13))
 (segment (start 60.539999 8.469999) (end 59.69 7.62) (width 0.25) (layer F.Cu) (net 6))
 (segment (start 61.315011 9.245011) (end 60.539999 8.469999) (width 0.25) (layer F.Cu) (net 6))
 (segment (start 61.315011 13.614989) (end 61.315011 9.245011) (width 0.25) (layer F.Cu) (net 6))
 (segment (start 59.69 15.24) (end 61.315011 13.614989) (width 0.25) (layer F.Cu) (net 6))
 (segment (start 59.69 7.62) (end 57.15 7.62) (width 0.25) (layer F.Cu) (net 6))
 (segment (start 52.07 10.16) (end 52.07 7.62) (width 0.25) (layer F.Cu) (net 3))
 (segment (start 60.79 10.16) (end 59.69 10.16) (width 0.25) (layer F.Cu) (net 7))
 (segment (start 60.865001 10.235001) (end 60.79 10.16) (width 0.25) (layer F.Cu) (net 7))
 (segment (start 60.254001 13.875001) (end 60.865001 13.264001) (width 0.25) (layer F.Cu) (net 7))
 (segment (start 59.315997 13.875001) (end 60.254001 13.875001) (width 0.25) (layer F.Cu) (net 7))
 (segment (start 58.514999 14.675999) (end 59.315997 13.875001) (width 0.25) (layer F.Cu) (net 7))
 (segment (start 58.514999 17.515001) (end 58.514999 14.675999) (width 0.25) (layer F.Cu) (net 7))
 (segment (start 58.25 17.78) (end 58.514999 17.515001) (width 0.25) (layer F.Cu) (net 7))
 (segment (start 60.865001 13.264001) (end 60.865001 10.235001) (width 0.25) (layer F.Cu) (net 7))
 (segment (start 57.15 17.78) (end 58.25 17.78) (width 0.25) (layer F.Cu) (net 7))
 (segment (start 59.69 10.16) (end 57.15 10.16) (width 0.25) (layer F.Cu) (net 7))
 (segment (start 32.549999 21.119999) (end 31.75 20.32) (width 0.25) (layer F.Cu) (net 7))
 (segment (start 40.784999 21.445001) (end 32.875001 21.445001) (width 0.25) (layer F.Cu) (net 7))
 (segment (start 32.875001 21.445001) (end 32.549999 21.119999) (width 0.25) (layer F.Cu) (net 7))
 (segment (start 41.91 20.32) (end 40.784999 21.445001) (width 0.25) (layer F.Cu) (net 7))
 (segment (start 56.05 17.78) (end 57.15 17.78) (width 0.25) (layer F.Cu) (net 7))
 (segment (start 48.835997 21.445001) (end 52.500998 17.78) (width 0.25) (layer F.Cu) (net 7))
 (segment (start 52.500998 17.78) (end 56.05 17.78) (width 0.25) (layer F.Cu) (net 7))
 (segment (start 43.035001 21.445001) (end 48.835997 21.445001) (width 0.25) (layer F.Cu) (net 7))
 (segment (start 41.91 20.32) (end 43.035001 21.445001) (width 0.25) (layer F.Cu) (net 7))
 (segment (start 31.75 20.32) (end 26.67 20.32) (width 0.25) (layer F.Cu) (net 7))
 (segment (start 25.870001 21.119999) (end 26.67 20.32) (width 0.25) (layer F.Cu) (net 7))
 (segment (start 25.544999 21.445001) (end 25.870001 21.119999) (width 0.25) (layer F.Cu) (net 7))
 (segment (start 22.715001 21.445001) (end 25.544999 21.445001) (width 0.25) (layer F.Cu) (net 7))
 (segment (start 21.59 20.32) (end 22.715001 21.445001) (width 0.25) (layer F.Cu) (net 7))
 (segment (start 6.914001 3.904999) (end 3.885001 3.904999) (width 0.25) (layer F.Cu) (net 7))
 (segment (start 6.974003 3.965001) (end 6.914001 3.904999) (width 0.25) (layer F.Cu) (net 7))
 (segment (start 3.81 3.98) (end 3.81 5.08) (width 0.25) (layer F.Cu) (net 7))
 (segment (start 15.084999 3.965001) (end 6.974003 3.965001) (width 0.25) (layer F.Cu) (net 7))
 (segment (start 3.885001 3.904999) (end 3.81 3.98) (width 0.25) (layer F.Cu) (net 7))
 (segment (start 16.51 2.54) (end 15.084999 3.965001) (width 0.25) (layer F.Cu) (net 7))
 (segment (start 3.81 5.08) (end 3.81 7.62) (width 0.25) (layer F.Cu) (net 7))
 (segment (start 3.81 7.62) (end 3.81 10.16) (width 0.25) (layer F.Cu) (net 7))
 (segment (start 3.81 10.16) (end 3.81 12.7) (width 0.25) (layer F.Cu) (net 7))
 (segment (start 6.035999 21.745001) (end 2.54 18.249002) (width 0.25) (layer F.Cu) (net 7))
 (segment (start 12.114001 21.745001) (end 6.035999 21.745001) (width 0.25) (layer F.Cu) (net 7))
 (segment (start 14.664003 19.194999) (end 12.114001 21.745001) (width 0.25) (layer F.Cu) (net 7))
 (segment (start 21.59 20.32) (end 20.464999 19.194999) (width 0.25) (layer F.Cu) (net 7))
 (segment (start 20.464999 19.194999) (end 14.664003 19.194999) (width 0.25) (layer F.Cu) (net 7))
 (segment (start 2.54 13.97) (end 3.81 12.7) (width 0.25) (layer F.Cu) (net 7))
 (segment (start 2.54 18.249002) (end 2.54 13.97) (width 0.25) (layer F.Cu) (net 7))
 (segment (start 6.35 7.62) (end 6.35 10.16) (width 0.25) (layer F.Cu) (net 14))
 (segment (start 8.89 10.16) (end 11.43 12.7) (width 0.25) (layer F.Cu) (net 14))
 (segment (start 6.35 10.16) (end 8.89 10.16) (width 0.25) (layer F.Cu) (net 14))
 (segment (start 11.43 13.8) (end 11.43 12.7) (width 0.25) (layer F.Cu) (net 14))
 (segment (start 11.90501 14.27501) (end 11.43 13.8) (width 0.25) (layer F.Cu) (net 14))
 (segment (start 22.55499 14.27501) (end 11.90501 14.27501) (width 0.25) (layer F.Cu) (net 14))
 (segment (start 24.13 12.7) (end 22.55499 14.27501) (width 0.25) (layer F.Cu) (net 14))
 (segment (start 53.17 15.24) (end 52.07 15.24) (width 0.25) (layer B.Cu) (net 14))
 (segment (start 53.245001 11.779997) (end 53.245001 15.164999) (width 0.25) (layer B.Cu) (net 14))
 (segment (start 56.039999 8.984999) (end 53.245001 11.779997) (width 0.25) (layer B.Cu) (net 14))
 (segment (start 57.524003 8.984999) (end 56.039999 8.984999) (width 0.25) (layer B.Cu) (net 14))
 (segment (start 58.325001 8.184001) (end 57.524003 8.984999) (width 0.25) (layer B.Cu) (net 14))
 (segment (start 58.325001 5.344999) (end 58.325001 8.184001) (width 0.25) (layer B.Cu) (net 14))
 (segment (start 53.245001 15.164999) (end 53.17 15.24) (width 0.25) (layer B.Cu) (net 14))
 (segment (start 58.59 5.08) (end 58.325001 5.344999) (width 0.25) (layer B.Cu) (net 14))
 (segment (start 59.69 5.08) (end 58.59 5.08) (width 0.25) (layer B.Cu) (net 14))
 (segment (start 26.67 15.24) (end 24.13 12.7) (width 0.25) (layer B.Cu) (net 14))
 (segment (start 52.07 15.24) (end 26.67 15.24) (width 0.25) (layer B.Cu) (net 14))
 (segment (start 11.43 10.16) (end 16.51 10.16) (width 0.25) (layer F.Cu) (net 22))
 (segment (start 46.99 17.78) (end 46.99 20.32) (width 0.25) (layer F.Cu) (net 5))
 (segment (start 52.07 12.7) (end 46.99 17.78) (width 0.25) (layer F.Cu) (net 5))
 (segment (start 37.629999 19.520001) (end 36.83 20.32) (width 0.25) (layer F.Cu) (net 5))
 (segment (start 37.955001 19.194999) (end 37.629999 19.520001) (width 0.25) (layer F.Cu) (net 5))
 (segment (start 45.864999 19.194999) (end 37.955001 19.194999) (width 0.25) (layer F.Cu) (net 5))
 (segment (start 46.99 20.32) (end 45.864999 19.194999) (width 0.25) (layer F.Cu) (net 5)))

